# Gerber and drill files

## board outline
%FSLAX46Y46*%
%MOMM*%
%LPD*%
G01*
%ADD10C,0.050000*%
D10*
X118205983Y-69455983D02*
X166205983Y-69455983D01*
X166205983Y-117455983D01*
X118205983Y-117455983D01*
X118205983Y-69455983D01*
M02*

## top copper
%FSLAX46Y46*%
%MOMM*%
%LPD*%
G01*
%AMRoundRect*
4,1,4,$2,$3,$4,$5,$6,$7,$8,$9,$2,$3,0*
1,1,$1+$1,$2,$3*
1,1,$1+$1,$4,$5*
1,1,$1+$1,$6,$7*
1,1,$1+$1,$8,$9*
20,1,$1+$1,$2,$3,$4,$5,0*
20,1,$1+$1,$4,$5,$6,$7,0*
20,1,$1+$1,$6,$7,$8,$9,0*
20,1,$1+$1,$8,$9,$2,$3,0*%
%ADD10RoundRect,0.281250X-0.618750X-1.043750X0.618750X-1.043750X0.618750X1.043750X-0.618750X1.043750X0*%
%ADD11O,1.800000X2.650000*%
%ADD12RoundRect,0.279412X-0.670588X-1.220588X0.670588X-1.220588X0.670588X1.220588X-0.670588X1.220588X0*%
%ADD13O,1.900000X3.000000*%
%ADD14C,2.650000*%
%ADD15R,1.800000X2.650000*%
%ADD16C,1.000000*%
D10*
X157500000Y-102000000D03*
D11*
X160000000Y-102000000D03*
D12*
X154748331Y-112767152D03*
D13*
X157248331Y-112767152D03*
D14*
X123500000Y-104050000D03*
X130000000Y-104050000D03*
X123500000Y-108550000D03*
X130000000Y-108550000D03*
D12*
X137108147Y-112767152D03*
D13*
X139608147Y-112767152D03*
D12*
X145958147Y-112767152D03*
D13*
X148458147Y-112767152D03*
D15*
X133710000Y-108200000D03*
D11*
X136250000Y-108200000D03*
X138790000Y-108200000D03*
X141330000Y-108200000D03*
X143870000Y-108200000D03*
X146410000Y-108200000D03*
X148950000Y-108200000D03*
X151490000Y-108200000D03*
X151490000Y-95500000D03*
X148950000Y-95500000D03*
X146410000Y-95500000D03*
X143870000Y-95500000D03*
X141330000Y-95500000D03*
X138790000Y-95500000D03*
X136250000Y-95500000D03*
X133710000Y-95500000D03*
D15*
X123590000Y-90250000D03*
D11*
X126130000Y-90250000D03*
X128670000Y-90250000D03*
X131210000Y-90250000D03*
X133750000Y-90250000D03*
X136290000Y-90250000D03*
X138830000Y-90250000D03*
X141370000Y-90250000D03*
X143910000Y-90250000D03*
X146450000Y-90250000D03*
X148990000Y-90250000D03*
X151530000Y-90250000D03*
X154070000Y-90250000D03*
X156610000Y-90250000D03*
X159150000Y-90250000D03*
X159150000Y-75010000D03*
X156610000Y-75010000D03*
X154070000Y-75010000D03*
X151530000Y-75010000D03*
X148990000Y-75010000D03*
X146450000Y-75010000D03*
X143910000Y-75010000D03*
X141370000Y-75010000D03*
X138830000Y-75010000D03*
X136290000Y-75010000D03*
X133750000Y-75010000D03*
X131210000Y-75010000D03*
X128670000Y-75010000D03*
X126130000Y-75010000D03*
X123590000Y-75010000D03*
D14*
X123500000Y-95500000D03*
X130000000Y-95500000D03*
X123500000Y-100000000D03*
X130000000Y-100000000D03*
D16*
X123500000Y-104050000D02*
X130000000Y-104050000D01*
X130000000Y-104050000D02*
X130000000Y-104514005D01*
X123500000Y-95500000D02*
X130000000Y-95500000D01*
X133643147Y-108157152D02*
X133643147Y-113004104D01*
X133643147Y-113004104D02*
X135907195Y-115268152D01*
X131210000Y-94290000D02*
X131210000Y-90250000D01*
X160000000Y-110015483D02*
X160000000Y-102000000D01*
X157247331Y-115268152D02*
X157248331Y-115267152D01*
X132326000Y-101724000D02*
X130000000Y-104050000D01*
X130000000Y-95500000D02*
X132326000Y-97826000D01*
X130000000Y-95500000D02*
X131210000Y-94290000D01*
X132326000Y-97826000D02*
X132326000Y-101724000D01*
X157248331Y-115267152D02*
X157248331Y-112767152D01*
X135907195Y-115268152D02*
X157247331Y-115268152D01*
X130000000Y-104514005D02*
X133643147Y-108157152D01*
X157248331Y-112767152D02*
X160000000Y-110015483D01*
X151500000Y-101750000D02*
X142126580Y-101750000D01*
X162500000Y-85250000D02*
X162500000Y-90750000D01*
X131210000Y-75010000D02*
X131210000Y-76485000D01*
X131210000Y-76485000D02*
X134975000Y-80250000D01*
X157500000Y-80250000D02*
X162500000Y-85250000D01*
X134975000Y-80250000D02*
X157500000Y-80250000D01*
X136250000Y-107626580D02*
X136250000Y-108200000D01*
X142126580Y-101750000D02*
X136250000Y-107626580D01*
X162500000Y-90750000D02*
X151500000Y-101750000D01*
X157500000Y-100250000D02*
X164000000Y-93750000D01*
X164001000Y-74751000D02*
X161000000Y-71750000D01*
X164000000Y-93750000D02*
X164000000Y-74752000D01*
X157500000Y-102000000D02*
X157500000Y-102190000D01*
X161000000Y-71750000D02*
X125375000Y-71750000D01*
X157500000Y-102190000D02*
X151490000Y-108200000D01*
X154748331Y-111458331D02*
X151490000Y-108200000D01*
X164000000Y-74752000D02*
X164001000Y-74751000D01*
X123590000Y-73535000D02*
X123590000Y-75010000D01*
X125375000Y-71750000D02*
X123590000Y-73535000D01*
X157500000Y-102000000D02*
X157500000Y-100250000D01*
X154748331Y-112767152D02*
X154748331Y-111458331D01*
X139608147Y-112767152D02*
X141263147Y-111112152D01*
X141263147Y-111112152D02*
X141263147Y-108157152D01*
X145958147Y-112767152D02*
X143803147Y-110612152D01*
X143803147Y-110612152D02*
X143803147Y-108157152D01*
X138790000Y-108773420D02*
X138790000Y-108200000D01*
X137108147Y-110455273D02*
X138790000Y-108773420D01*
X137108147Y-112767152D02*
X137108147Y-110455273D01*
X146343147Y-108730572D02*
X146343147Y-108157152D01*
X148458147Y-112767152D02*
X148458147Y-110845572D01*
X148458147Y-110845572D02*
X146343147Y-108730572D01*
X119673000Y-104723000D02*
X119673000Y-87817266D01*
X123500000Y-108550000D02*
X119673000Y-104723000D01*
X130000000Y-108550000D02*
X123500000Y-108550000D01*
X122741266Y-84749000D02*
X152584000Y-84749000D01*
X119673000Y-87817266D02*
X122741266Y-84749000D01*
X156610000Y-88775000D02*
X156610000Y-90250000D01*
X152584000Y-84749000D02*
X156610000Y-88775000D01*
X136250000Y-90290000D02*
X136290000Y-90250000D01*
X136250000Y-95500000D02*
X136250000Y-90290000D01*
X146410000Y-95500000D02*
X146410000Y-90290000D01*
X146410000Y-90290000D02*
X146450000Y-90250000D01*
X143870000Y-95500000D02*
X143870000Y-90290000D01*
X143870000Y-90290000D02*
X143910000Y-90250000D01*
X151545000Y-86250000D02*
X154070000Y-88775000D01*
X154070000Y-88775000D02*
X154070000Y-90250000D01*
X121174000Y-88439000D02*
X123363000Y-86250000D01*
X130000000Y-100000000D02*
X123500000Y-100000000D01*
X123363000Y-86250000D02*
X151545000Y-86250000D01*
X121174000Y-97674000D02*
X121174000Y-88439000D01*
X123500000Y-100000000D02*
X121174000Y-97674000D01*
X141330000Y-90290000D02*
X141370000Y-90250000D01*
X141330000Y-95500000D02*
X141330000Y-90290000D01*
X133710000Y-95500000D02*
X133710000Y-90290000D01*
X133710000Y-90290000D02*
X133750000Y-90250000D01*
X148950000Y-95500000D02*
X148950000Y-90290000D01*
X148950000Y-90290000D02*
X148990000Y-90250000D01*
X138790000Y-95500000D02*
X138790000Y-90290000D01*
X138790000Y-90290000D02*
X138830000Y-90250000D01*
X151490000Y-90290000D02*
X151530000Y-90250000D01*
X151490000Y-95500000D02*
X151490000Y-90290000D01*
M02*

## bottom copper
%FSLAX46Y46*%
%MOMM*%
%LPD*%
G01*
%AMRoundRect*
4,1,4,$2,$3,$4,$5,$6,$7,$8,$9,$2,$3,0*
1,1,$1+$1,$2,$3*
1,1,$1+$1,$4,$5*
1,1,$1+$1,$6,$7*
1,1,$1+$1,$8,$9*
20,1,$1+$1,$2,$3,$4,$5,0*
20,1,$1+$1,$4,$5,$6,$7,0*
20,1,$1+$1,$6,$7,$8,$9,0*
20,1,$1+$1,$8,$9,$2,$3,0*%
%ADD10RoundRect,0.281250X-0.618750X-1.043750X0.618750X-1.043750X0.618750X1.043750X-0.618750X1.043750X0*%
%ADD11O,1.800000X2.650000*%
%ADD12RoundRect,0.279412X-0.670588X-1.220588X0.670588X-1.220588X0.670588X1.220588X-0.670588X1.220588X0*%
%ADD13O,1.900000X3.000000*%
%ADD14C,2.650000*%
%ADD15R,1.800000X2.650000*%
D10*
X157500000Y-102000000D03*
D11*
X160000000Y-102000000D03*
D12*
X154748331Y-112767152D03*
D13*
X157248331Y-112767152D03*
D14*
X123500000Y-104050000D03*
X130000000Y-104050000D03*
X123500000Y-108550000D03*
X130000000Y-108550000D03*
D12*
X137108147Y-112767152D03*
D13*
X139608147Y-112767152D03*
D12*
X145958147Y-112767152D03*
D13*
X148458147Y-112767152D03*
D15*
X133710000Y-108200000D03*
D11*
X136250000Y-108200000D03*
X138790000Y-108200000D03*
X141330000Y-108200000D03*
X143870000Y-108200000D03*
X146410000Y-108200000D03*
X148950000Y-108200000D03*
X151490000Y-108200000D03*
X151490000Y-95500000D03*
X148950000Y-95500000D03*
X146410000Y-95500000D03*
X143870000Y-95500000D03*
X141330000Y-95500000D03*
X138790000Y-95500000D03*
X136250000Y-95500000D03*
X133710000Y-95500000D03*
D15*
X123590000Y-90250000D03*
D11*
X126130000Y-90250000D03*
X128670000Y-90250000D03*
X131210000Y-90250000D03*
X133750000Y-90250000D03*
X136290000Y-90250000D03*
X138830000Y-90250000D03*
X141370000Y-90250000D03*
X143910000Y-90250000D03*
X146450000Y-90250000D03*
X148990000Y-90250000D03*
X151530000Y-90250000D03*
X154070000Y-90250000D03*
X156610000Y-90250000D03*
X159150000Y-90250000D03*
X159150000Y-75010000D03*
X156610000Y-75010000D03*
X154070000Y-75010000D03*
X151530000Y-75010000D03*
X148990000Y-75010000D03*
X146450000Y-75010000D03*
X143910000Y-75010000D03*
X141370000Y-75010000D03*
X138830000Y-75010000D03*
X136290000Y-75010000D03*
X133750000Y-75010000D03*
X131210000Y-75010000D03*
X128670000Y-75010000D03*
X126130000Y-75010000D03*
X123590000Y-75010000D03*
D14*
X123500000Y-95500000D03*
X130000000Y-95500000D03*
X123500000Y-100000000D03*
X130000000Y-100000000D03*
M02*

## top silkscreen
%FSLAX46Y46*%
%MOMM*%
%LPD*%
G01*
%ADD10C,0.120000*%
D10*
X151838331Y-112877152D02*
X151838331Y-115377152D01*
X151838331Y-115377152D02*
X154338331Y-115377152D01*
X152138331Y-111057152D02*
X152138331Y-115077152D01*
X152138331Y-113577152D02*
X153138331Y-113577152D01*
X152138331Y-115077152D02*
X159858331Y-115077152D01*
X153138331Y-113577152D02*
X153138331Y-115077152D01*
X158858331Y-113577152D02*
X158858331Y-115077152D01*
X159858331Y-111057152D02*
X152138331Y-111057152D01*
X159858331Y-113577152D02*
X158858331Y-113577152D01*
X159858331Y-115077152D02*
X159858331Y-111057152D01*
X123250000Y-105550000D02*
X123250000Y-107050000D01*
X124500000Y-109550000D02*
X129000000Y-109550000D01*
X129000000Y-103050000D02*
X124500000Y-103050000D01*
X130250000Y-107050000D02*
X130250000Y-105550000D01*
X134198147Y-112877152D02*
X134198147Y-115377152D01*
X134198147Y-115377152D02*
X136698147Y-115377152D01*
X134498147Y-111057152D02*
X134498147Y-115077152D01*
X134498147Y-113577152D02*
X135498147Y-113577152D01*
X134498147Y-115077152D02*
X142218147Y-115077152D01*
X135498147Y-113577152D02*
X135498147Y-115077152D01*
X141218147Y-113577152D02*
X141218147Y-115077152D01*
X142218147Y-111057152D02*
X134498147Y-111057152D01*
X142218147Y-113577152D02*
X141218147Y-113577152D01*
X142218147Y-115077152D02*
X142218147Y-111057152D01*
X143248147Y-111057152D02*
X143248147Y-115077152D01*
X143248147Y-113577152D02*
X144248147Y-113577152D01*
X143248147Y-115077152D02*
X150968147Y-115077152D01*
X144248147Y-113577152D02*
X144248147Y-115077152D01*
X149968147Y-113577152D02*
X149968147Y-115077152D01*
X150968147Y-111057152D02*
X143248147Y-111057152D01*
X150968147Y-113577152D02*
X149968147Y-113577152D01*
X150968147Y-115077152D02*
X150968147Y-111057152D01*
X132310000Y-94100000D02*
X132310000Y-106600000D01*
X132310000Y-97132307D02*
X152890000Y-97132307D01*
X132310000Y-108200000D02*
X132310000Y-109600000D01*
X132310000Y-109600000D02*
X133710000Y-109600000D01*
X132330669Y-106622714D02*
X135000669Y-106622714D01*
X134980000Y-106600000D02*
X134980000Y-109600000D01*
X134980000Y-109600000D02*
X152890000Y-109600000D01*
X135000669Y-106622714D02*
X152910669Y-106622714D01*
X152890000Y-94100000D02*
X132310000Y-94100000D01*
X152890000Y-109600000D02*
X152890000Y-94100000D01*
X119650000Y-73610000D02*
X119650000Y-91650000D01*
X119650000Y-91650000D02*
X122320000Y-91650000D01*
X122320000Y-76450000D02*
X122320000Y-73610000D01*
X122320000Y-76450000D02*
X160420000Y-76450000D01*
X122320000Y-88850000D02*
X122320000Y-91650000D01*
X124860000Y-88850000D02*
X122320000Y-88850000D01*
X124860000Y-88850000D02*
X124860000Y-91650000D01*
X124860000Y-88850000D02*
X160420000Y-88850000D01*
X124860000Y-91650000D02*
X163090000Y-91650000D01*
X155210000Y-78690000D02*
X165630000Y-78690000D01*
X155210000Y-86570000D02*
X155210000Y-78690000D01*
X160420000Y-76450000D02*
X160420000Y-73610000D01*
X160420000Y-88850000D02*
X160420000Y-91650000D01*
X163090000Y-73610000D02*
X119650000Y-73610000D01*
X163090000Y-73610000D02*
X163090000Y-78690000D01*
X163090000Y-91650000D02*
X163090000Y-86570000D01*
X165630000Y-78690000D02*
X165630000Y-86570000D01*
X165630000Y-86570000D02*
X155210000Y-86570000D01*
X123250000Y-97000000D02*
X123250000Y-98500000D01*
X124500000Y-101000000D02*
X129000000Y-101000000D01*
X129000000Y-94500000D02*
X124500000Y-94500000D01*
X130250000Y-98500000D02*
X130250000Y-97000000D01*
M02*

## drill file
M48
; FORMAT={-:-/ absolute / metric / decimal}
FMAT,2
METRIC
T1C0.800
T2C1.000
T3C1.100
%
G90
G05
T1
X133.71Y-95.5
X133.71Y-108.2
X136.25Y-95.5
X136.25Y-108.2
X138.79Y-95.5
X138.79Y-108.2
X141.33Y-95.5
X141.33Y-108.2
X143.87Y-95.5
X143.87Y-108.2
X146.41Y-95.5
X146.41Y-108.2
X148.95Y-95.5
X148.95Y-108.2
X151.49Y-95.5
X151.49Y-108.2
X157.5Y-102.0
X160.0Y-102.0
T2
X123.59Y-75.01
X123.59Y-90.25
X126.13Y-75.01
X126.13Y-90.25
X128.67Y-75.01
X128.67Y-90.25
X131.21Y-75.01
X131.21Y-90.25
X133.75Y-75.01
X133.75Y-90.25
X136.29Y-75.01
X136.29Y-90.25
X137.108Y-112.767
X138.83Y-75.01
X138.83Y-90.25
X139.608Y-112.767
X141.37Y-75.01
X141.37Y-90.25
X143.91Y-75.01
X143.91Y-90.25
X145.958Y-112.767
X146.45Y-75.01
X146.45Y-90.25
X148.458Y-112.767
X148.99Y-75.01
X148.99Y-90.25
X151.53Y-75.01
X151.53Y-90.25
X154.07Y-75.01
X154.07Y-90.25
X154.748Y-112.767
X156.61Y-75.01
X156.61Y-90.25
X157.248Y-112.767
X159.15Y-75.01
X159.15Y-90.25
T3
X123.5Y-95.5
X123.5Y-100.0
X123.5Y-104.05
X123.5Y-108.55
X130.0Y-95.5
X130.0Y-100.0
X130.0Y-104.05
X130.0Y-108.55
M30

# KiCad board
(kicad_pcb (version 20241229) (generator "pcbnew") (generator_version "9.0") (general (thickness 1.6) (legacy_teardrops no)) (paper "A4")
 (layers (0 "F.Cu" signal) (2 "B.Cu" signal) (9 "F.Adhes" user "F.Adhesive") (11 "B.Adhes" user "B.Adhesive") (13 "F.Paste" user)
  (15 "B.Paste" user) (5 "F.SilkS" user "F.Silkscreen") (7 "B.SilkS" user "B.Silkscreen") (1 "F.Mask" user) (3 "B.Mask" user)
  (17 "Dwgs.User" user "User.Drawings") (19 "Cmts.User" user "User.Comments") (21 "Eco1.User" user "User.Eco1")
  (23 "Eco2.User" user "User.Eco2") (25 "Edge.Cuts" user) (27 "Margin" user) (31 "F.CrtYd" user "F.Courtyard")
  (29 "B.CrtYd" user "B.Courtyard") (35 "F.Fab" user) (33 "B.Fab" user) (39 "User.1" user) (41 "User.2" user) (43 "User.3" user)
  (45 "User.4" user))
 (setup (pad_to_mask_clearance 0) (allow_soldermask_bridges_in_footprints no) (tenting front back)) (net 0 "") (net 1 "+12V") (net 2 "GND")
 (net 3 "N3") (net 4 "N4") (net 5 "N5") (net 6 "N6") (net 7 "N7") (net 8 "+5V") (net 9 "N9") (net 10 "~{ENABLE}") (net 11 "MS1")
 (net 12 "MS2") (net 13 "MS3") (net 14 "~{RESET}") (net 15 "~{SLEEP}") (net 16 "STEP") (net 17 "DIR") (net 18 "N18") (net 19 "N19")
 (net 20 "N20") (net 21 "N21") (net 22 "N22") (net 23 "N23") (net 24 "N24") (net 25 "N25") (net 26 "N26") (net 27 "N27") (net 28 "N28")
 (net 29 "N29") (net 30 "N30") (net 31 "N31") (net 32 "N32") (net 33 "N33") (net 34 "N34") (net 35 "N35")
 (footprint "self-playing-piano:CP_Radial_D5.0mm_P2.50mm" (layer "F.Cu") (at 157.5 102)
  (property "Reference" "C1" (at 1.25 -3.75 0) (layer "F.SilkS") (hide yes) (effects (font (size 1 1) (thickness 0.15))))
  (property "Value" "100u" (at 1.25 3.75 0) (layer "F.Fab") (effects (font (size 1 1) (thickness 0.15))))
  (pad "1" thru_hole roundrect (at 0 0) (size 1.8 2.65) (drill 0.8) (layers "*.Cu" "*.Mask") (remove_unused_layers no)
   (roundrect_rratio 0.15625) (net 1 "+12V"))
  (pad "2" thru_hole oval (at 2.5 0) (size 1.8 2.65) (drill 0.8) (layers "*.Cu" "*.Mask") (remove_unused_layers no) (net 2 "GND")))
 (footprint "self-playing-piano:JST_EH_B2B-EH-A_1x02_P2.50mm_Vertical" (layer "F.Cu") (at 154.748331 112.767152)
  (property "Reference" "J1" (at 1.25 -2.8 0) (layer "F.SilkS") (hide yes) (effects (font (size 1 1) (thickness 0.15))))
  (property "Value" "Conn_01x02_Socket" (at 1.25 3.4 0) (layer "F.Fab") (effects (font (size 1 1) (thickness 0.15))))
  (fp_line (start -2.91 0.11) (end -2.91 2.61) (stroke (width 0.12) (type solid)) (layer "F.SilkS"))
  (fp_line (start -2.91 2.61) (end -0.41 2.61) (stroke (width 0.12) (type solid)) (layer "F.SilkS"))
  (fp_line (start -2.61 -1.71) (end -2.61 2.31) (stroke (width 0.12) (type solid)) (layer "F.SilkS"))
  (fp_line (start -2.61 0.81) (end -1.61 0.81) (stroke (width 0.12) (type solid)) (layer "F.SilkS"))
  (fp_line (start -2.61 2.31) (end 5.11 2.31) (stroke (width 0.12) (type solid)) (layer "F.SilkS"))
  (fp_line (start -1.61 0.81) (end -1.61 2.31) (stroke (width 0.12) (type solid)) (layer "F.SilkS"))
  (fp_line (start 4.11 0.81) (end 4.11 2.31) (stroke (width 0.12) (type solid)) (layer "F.SilkS"))
  (fp_line (start 5.11 -1.71) (end -2.61 -1.71) (stroke (width 0.12) (type solid)) (layer "F.SilkS"))
  (fp_line (start 5.11 0.81) (end 4.11 0.81) (stroke (width 0.12) (type solid)) (layer "F.SilkS"))
  (fp_line (start 5.11 2.31) (end 5.11 -1.71) (stroke (width 0.12) (type solid)) (layer "F.SilkS"))
  (pad "1" thru_hole roundrect (at 0 0) (size 1.9 3) (drill 1) (layers "*.Cu" "*.Mask") (remove_unused_layers no)
   (roundrect_rratio 0.147059) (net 1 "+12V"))
  (pad "2" thru_hole oval (at 2.5 0) (size 1.9 3) (drill 1) (layers "*.Cu" "*.Mask") (remove_unused_layers no) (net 2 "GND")))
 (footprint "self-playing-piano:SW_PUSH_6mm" (layer "F.Cu") (at 123.5 104.05)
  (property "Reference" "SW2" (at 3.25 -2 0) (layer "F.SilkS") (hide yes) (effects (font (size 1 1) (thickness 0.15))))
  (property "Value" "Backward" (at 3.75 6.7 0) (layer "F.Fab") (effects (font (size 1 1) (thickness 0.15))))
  (fp_line (start -0.25 1.5) (end -0.25 3) (stroke (width 0.12) (type solid)) (layer "F.SilkS"))
  (fp_line (start 1 5.5) (end 5.5 5.5) (stroke (width 0.12) (type solid)) (layer "F.SilkS"))
  (fp_line (start 5.5 -1) (end 1 -1) (stroke (width 0.12) (type solid)) (layer "F.SilkS"))
  (fp_line (start 6.75 3) (end 6.75 1.5) (stroke (width 0.12) (type solid)) (layer "F.SilkS"))
  (pad "1" thru_hole circle (at 0 0 90) (size 2.65 2.65) (drill 1.1) (layers "*.Cu" "*.Mask") (remove_unused_layers no) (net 2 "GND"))
  (pad "1" thru_hole circle (at 6.5 0 90) (size 2.65 2.65) (drill 1.1) (layers "*.Cu" "*.Mask") (remove_unused_layers no) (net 2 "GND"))
  (pad "2" thru_hole circle (at 0 4.5 90) (size 2.65 2.65) (drill 1.1) (layers "*.Cu" "*.Mask") (remove_unused_layers no) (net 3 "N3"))
  (pad "2" thru_hole circle (at 6.5 4.5 90) (size 2.65 2.65) (drill 1.1) (layers "*.Cu" "*.Mask") (remove_unused_layers no) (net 3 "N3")))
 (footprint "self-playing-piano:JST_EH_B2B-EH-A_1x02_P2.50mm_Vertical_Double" (layer "F.Cu") (at 137.108147 112.767152)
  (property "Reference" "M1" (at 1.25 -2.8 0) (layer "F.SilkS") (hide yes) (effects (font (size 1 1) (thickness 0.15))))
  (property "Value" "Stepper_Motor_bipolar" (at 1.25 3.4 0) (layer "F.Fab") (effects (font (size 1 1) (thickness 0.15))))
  (fp_line (start -2.91 0.11) (end -2.91 2.61) (stroke (width 0.12) (type solid)) (layer "F.SilkS"))
  (fp_line (start -2.91 2.61) (end -0.41 2.61) (stroke (width 0.12) (type solid)) (layer "F.SilkS"))
  (fp_line (start -2.61 -1.71) (end -2.61 2.31) (stroke (width 0.12) (type solid)) (layer "F.SilkS"))
  (fp_line (start -2.61 0.81) (end -1.61 0.81) (stroke (width 0.12) (type solid)) (layer "F.SilkS"))
  (fp_line (start -2.61 2.31) (end 5.11 2.31) (stroke (width 0.12) (type solid)) (layer "F.SilkS"))
  (fp_line (start -1.61 0.81) (end -1.61 2.31) (stroke (width 0.12) (type solid)) (layer "F.SilkS"))
  (fp_line (start 4.11 0.81) (end 4.11 2.31) (stroke (width 0.12) (type solid)) (layer "F.SilkS"))
  (fp_line (start 5.11 -1.71) (end -2.61 -1.71) (stroke (width 0.12) (type solid)) (layer "F.SilkS"))
  (fp_line (start 5.11 0.81) (end 4.11 0.81) (stroke (width 0.12) (type solid)) (layer "F.SilkS"))
  (fp_line (start 5.11 2.31) (end 5.11 -1.71) (stroke (width 0.12) (type solid)) (layer "F.SilkS"))
  (fp_line (start 6.14 -1.71) (end 6.14 2.31) (stroke (width 0.12) (type solid)) (layer "F.SilkS"))
  (fp_line (start 6.14 0.81) (end 7.14 0.81) (stroke (width 0.12) (type solid)) (layer "F.SilkS"))
  (fp_line (start 6.14 2.31) (end 13.86 2.31) (stroke (width 0.12) (type solid)) (layer "F.SilkS"))
  (fp_line (start 7.14 0.81) (end 7.14 2.31) (stroke (width 0.12) (type solid)) (layer "F.SilkS"))
  (fp_line (start 12.86 0.81) (end 12.86 2.31) (stroke (width 0.12) (type solid)) (layer "F.SilkS"))
  (fp_line (start 13.86 -1.71) (end 6.14 -1.71) (stroke (width 0.12) (type solid)) (layer "F.SilkS"))
  (fp_line (start 13.86 0.81) (end 12.86 0.81) (stroke (width 0.12) (type solid)) (layer "F.SilkS"))
  (fp_line (start 13.86 2.31) (end 13.86 -1.71) (stroke (width 0.12) (type solid)) (layer "F.SilkS"))
  (pad "1" thru_hole roundrect (at 0 0) (size 1.9 3) (drill 1) (layers "*.Cu" "*.Mask") (remove_unused_layers no)
   (roundrect_rratio 0.147059) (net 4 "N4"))
  (pad "2" thru_hole oval (at 2.5 0) (size 1.9 3) (drill 1) (layers "*.Cu" "*.Mask") (remove_unused_layers no) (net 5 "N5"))
  (pad "3" thru_hole roundrect (at 8.85 0) (size 1.9 3) (drill 1) (layers "*.Cu" "*.Mask") (remove_unused_layers no)
   (roundrect_rratio 0.147059) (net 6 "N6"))
  (pad "4" thru_hole oval (at 11.35 0) (size 1.9 3) (drill 1) (layers "*.Cu" "*.Mask") (remove_unused_layers no) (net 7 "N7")))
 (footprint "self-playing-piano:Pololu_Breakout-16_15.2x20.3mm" (layer "F.Cu") (at 133.71 108.2 90)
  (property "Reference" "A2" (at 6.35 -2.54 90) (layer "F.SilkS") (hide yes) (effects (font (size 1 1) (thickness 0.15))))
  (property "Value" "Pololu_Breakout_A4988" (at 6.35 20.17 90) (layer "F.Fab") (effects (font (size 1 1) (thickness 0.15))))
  (fp_line (start 14.1 -1.4) (end 1.6 -1.4) (stroke (width 0.12) (type solid)) (layer "F.SilkS"))
  (fp_line (start 11.067693 -1.4) (end 11.067693 19.18) (stroke (width 0.12) (type solid)) (layer "F.SilkS"))
  (fp_line (start 0 -1.4) (end -1.4 -1.4) (stroke (width 0.12) (type solid)) (layer "F.SilkS"))
  (fp_line (start -1.4 -1.4) (end -1.4 0) (stroke (width 0.12) (type solid)) (layer "F.SilkS"))
  (fp_line (start 1.577286 -1.379331) (end 1.577286 1.290669) (stroke (width 0.12) (type solid)) (layer "F.SilkS"))
  (fp_line (start 1.6 1.27) (end -1.4 1.27) (stroke (width 0.12) (type solid)) (layer "F.SilkS"))
  (fp_line (start -1.4 1.27) (end -1.4 19.18) (stroke (width 0.12) (type solid)) (layer "F.SilkS"))
  (fp_line (start 1.577286 1.290669) (end 1.577286 19.200669) (stroke (width 0.12) (type solid)) (layer "F.SilkS"))
  (fp_line (start 14.1 19.18) (end 14.1 -1.4) (stroke (width 0.12) (type solid)) (layer "F.SilkS"))
  (fp_line (start -1.4 19.18) (end 14.1 19.18) (stroke (width 0.12) (type solid)) (layer "F.SilkS"))
  (pad "1" thru_hole rect (at 0 0 90) (size 2.65 1.8) (drill 0.8) (layers "*.Cu" "*.Mask") (remove_unused_layers no) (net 2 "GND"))
  (pad "2" thru_hole oval (at 0 2.54 90) (size 2.65 1.8) (drill 0.8) (layers "*.Cu" "*.Mask") (remove_unused_layers no) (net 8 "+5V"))
  (pad "3" thru_hole oval (at 0 5.08 90) (size 2.65 1.8) (drill 0.8) (layers "*.Cu" "*.Mask") (remove_unused_layers no) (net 4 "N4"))
  (pad "4" thru_hole oval (at 0 7.62 90) (size 2.65 1.8) (drill 0.8) (layers "*.Cu" "*.Mask") (remove_unused_layers no) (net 5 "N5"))
  (pad "5" thru_hole oval (at 0 10.16 90) (size 2.65 1.8) (drill 0.8) (layers "*.Cu" "*.Mask") (remove_unused_layers no) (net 6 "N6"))
  (pad "6" thru_hole oval (at 0 12.7 90) (size 2.65 1.8) (drill 0.8) (layers "*.Cu" "*.Mask") (remove_unused_layers no) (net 7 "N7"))
  (pad "7" thru_hole oval (at 0 15.24 90) (size 2.65 1.8) (drill 0.8) (layers "*.Cu" "*.Mask") (remove_unused_layers no) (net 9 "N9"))
  (pad "8" thru_hole oval (at 0 17.78 90) (size 2.65 1.8) (drill 0.8) (layers "*.Cu" "*.Mask") (remove_unused_layers no) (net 1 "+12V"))
  (pad "9" thru_hole oval (at 12.7 17.78 90) (size 2.65 1.8) (drill 0.8) (layers "*.Cu" "*.Mask") (remove_unused_layers no)
   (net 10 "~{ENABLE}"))
  (pad "10" thru_hole oval (at 12.7 15.24 90) (size 2.65 1.8) (drill 0.8) (layers "*.Cu" "*.Mask") (remove_unused_layers no) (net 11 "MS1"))
  (pad "11" thru_hole oval (at 12.7 12.7 90) (size 2.65 1.8) (drill 0.8) (layers "*.Cu" "*.Mask") (remove_unused_layers no) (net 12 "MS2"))
  (pad "12" thru_hole oval (at 12.7 10.16 90) (size 2.65 1.8) (drill 0.8) (layers "*.Cu" "*.Mask") (remove_unused_layers no) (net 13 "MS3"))
  (pad "13" thru_hole oval (at 12.7 7.62 90) (size 2.65 1.8) (drill 0.8) (layers "*.Cu" "*.Mask") (remove_unused_layers no)
   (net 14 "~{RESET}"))
  (pad "14" thru_hole oval (at 12.7 5.08 90) (size 2.65 1.8) (drill 0.8) (layers "*.Cu" "*.Mask") (remove_unused_layers no)
   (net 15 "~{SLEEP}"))
  (pad "15" thru_hole oval (at 12.7 2.54 90) (size 2.65 1.8) (drill 0.8) (layers "*.Cu" "*.Mask") (remove_unused_layers no) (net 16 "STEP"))
  (pad "16" thru_hole oval (at 12.7 0 90) (size 2.65 1.8) (drill 0.8) (layers "*.Cu" "*.Mask") (remove_unused_layers no) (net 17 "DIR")))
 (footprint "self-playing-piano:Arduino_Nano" (layer "F.Cu") (at 123.59 90.25 90)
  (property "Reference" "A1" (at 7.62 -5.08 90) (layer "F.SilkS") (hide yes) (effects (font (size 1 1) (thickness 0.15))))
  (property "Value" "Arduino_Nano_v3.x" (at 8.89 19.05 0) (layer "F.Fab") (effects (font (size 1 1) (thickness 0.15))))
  (fp_line (start 16.64 -3.94) (end -1.4 -3.94) (stroke (width 0.12) (type solid)) (layer "F.SilkS"))
  (fp_line (start -1.4 -3.94) (end -1.4 -1.27) (stroke (width 0.12) (type solid)) (layer "F.SilkS"))
  (fp_line (start 13.8 -1.27) (end 16.64 -1.27) (stroke (width 0.12) (type solid)) (layer "F.SilkS"))
  (fp_line (start 13.8 -1.27) (end 13.8 36.83) (stroke (width 0.12) (type solid)) (layer "F.SilkS"))
  (fp_line (start 1.4 -1.27) (end -1.4 -1.27) (stroke (width 0.12) (type solid)) (layer "F.SilkS"))
  (fp_line (start 1.4 1.27) (end 1.4 -1.27) (stroke (width 0.12) (type solid)) (layer "F.SilkS"))
  (fp_line (start 1.4 1.27) (end -1.4 1.27) (stroke (width 0.12) (type solid)) (layer "F.SilkS"))
  (fp_line (start 1.4 1.27) (end 1.4 36.83) (stroke (width 0.12) (type solid)) (layer "F.SilkS"))
  (fp_line (start -1.4 1.27) (end -1.4 39.5) (stroke (width 0.12) (type solid)) (layer "F.SilkS"))
  (fp_line (start 11.56 31.62) (end 11.56 42.04) (stroke (width 0.12) (type solid)) (layer "F.SilkS"))
  (fp_line (start 3.68 31.62) (end 11.56 31.62) (stroke (width 0.12) (type solid)) (layer "F.SilkS"))
  (fp_line (start 13.8 36.83) (end 16.64 36.83) (stroke (width 0.12) (type solid)) (layer "F.SilkS"))
  (fp_line (start 1.4 36.83) (end -1.4 36.83) (stroke (width 0.12) (type solid)) (layer "F.SilkS"))
  (fp_line (start 16.64 39.5) (end 16.64 -3.94) (stroke (width 0.12) (type solid)) (layer "F.SilkS"))
  (fp_line (start 16.64 39.5) (end 11.56 39.5) (stroke (width 0.12) (type solid)) (layer "F.SilkS"))
  (fp_line (start -1.4 39.5) (end 3.68 39.5) (stroke (width 0.12) (type solid)) (layer "F.SilkS"))
  (fp_line (start 11.56 42.04) (end 3.68 42.04) (stroke (width 0.12) (type solid)) (layer "F.SilkS"))
  (fp_line (start 3.68 42.04) (end 3.68 31.62) (stroke (width 0.12) (type solid)) (layer "F.SilkS"))
  (pad "1" thru_hole rect (at 0 0 90) (size 2.65 1.8) (drill 1) (layers "*.Cu" "*.Mask") (remove_unused_layers no) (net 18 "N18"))
  (pad "2" thru_hole oval (at 0 2.54 90) (size 2.65 1.8) (drill 1) (layers "*.Cu" "*.Mask") (remove_unused_layers no) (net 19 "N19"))
  (pad "3" thru_hole oval (at 0 5.08 90) (size 2.65 1.8) (drill 1) (layers "*.Cu" "*.Mask") (remove_unused_layers no) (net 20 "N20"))
  (pad "4" thru_hole oval (at 0 7.62 90) (size 2.65 1.8) (drill 1) (layers "*.Cu" "*.Mask") (remove_unused_layers no) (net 2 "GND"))
  (pad "5" thru_hole oval (at 0 10.16 90) (size 2.65 1.8) (drill 1) (layers "*.Cu" "*.Mask") (remove_unused_layers no) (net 17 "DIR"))
  (pad "6" thru_hole oval (at 0 12.7 90) (size 2.65 1.8) (drill 1) (layers "*.Cu" "*.Mask") (remove_unused_layers no) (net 16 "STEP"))
  (pad "7" thru_hole oval (at 0 15.24 90) (size 2.65 1.8) (drill 1) (layers "*.Cu" "*.Mask") (remove_unused_layers no) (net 15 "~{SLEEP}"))
  (pad "8" thru_hole oval (at 0 17.78 90) (size 2.65 1.8) (drill 1) (layers "*.Cu" "*.Mask") (remove_unused_layers no) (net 14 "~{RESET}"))
  (pad "9" thru_hole oval (at 0 20.32 90) (size 2.65 1.8) (drill 1) (layers "*.Cu" "*.Mask") (remove_unused_layers no) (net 13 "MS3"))
  (pad "10" thru_hole oval (at 0 22.86 90) (size 2.65 1.8) (drill 1) (layers "*.Cu" "*.Mask") (remove_unused_layers no) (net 12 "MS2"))
  (pad "11" thru_hole oval (at 0 25.4 90) (size 2.65 1.8) (drill 1) (layers "*.Cu" "*.Mask") (remove_unused_layers no) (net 11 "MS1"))
  (pad "12" thru_hole oval (at 0 27.94 90) (size 2.65 1.8) (drill 1) (layers "*.Cu" "*.Mask") (remove_unused_layers no) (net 10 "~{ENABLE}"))
  (pad "13" thru_hole oval (at 0 30.48 90) (size 2.65 1.8) (drill 1) (layers "*.Cu" "*.Mask") (remove_unused_layers no) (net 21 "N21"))
  (pad "14" thru_hole oval (at 0 33.02 90) (size 2.65 1.8) (drill 1) (layers "*.Cu" "*.Mask") (remove_unused_layers no) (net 3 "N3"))
  (pad "15" thru_hole oval (at 0 35.56 90) (size 2.65 1.8) (drill 1) (layers "*.Cu" "*.Mask") (remove_unused_layers no) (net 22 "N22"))
  (pad "16" thru_hole oval (at 15.24 35.56 90) (size 2.65 1.8) (drill 1) (layers "*.Cu" "*.Mask") (remove_unused_layers no) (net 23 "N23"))
  (pad "17" thru_hole oval (at 15.24 33.02 90) (size 2.65 1.8) (drill 1) (layers "*.Cu" "*.Mask") (remove_unused_layers no) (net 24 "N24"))
  (pad "18" thru_hole oval (at 15.24 30.48 90) (size 2.65 1.8) (drill 1) (layers "*.Cu" "*.Mask") (remove_unused_layers no) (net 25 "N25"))
  (pad "19" thru_hole oval (at 15.24 27.94 90) (size 2.65 1.8) (drill 1) (layers "*.Cu" "*.Mask") (remove_unused_layers no) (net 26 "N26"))
  (pad "20" thru_hole oval (at 15.24 25.4 90) (size 2.65 1.8) (drill 1) (layers "*.Cu" "*.Mask") (remove_unused_layers no) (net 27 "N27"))
  (pad "21" thru_hole oval (at 15.24 22.86 90) (size 2.65 1.8) (drill 1) (layers "*.Cu" "*.Mask") (remove_unused_layers no) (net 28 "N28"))
  (pad "22" thru_hole oval (at 15.24 20.32 90) (size 2.65 1.8) (drill 1) (layers "*.Cu" "*.Mask") (remove_unused_layers no) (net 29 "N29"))
  (pad "23" thru_hole oval (at 15.24 17.78 90) (size 2.65 1.8) (drill 1) (layers "*.Cu" "*.Mask") (remove_unused_layers no) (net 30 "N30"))
  (pad "24" thru_hole oval (at 15.24 15.24 90) (size 2.65 1.8) (drill 1) (layers "*.Cu" "*.Mask") (remove_unused_layers no) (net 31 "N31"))
  (pad "25" thru_hole oval (at 15.24 12.7 90) (size 2.65 1.8) (drill 1) (layers "*.Cu" "*.Mask") (remove_unused_layers no) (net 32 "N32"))
  (pad "26" thru_hole oval (at 15.24 10.16 90) (size 2.65 1.8) (drill 1) (layers "*.Cu" "*.Mask") (remove_unused_layers no) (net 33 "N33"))
  (pad "27" thru_hole oval (at 15.24 7.62 90) (size 2.65 1.8) (drill 1) (layers "*.Cu" "*.Mask") (remove_unused_layers no) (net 8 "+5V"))
  (pad "28" thru_hole oval (at 15.24 5.08 90) (size 2.65 1.8) (drill 1) (layers "*.Cu" "*.Mask") (remove_unused_layers no) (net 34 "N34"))
  (pad "29" thru_hole oval (at 15.24 2.54 90) (size 2.65 1.8) (drill 1) (layers "*.Cu" "*.Mask") (remove_unused_layers no) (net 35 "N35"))
  (pad "30" thru_hole oval (at 15.24 0 90) (size 2.65 1.8) (drill 1) (layers "*.Cu" "*.Mask") (remove_unused_layers no) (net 1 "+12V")))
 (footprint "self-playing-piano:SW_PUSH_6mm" (layer "F.Cu") (at 123.5 95.5)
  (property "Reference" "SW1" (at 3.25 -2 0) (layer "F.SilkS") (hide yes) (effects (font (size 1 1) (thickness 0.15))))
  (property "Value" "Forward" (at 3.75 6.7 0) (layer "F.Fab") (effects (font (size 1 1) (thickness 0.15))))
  (fp_line (start -0.25 1.5) (end -0.25 3) (stroke (width 0.12) (type solid)) (layer "F.SilkS"))
  (fp_line (start 1 5.5) (end 5.5 5.5) (stroke (width 0.12) (type solid)) (layer "F.SilkS"))
  (fp_line (start 5.5 -1) (end 1 -1) (stroke (width 0.12) (type solid)) (layer "F.SilkS"))
  (fp_line (start 6.75 3) (end 6.75 1.5) (stroke (width 0.12) (type solid)) (layer "F.SilkS"))
  (pad "1" thru_hole circle (at 0 0 90) (size 2.65 2.65) (drill 1.1) (layers "*.Cu" "*.Mask") (remove_unused_layers no) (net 2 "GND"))
  (pad "1" thru_hole circle (at 6.5 0 90) (size 2.65 2.65) (drill 1.1) (layers "*.Cu" "*.Mask") (remove_unused_layers no) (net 2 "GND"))
  (pad "2" thru_hole circle (at 0 4.5 90) (size 2.65 2.65) (drill 1.1) (layers "*.Cu" "*.Mask") (remove_unused_layers no) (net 21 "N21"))
  (pad "2" thru_hole circle (at 6.5 4.5 90) (size 2.65 2.65) (drill 1.1) (layers "*.Cu" "*.Mask") (remove_unused_layers no) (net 21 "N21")))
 (gr_rect (start 118.205983 69.455983) (end 166.205983 117.455983) (stroke (width 0.05) (type default)) (fill no) (layer "Edge.Cuts"))
 (segment (start 123.5 104.05) (end 130 104.05) (width 1) (layer "F.Cu") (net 2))
 (segment (start 130 104.05) (end 130 104.514005) (width 1) (layer "F.Cu") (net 2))
 (segment (start 123.5 95.5) (end 130 95.5) (width 1) (layer "F.Cu") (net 2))
 (segment (start 133.643147 108.157152) (end 133.643147 113.004104) (width 1) (layer "F.Cu") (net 2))
 (segment (start 133.643147 113.004104) (end 135.907195 115.268152) (width 1) (layer "F.Cu") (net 2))
 (segment (start 131.21 94.29) (end 131.21 90.25) (width 1) (layer "F.Cu") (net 2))
 (segment (start 160 110.015483) (end 160 102) (width 1) (layer "F.Cu") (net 2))
 (segment (start 157.247331 115.268152) (end 157.248331 115.267152) (width 1) (layer "F.Cu") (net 2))
 (segment (start 132.326 101.724) (end 130 104.05) (width 1) (layer "F.Cu") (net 2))
 (segment (start 130 95.5) (end 132.326 97.826) (width 1) (layer "F.Cu") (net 2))
 (segment (start 130 95.5) (end 131.21 94.29) (width 1) (layer "F.Cu") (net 2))
 (segment (start 132.326 97.826) (end 132.326 101.724) (width 1) (layer "F.Cu") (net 2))
 (segment (start 157.248331 115.267152) (end 157.248331 112.767152) (width 1) (layer "F.Cu") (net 2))
 (segment (start 135.907195 115.268152) (end 157.247331 115.268152) (width 1) (layer "F.Cu") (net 2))
 (segment (start 130 104.514005) (end 133.643147 108.157152) (width 1) (layer "F.Cu") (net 2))
 (segment (start 157.248331 112.767152) (end 160 110.015483) (width 1) (layer "F.Cu") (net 2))
 (segment (start 151.5 101.75) (end 142.12658 101.75) (width 1) (layer "F.Cu") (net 8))
 (segment (start 162.5 85.25) (end 162.5 90.75) (width 1) (layer "F.Cu") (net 8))
 (segment (start 131.21 75.01) (end 131.21 76.485) (width 1) (layer "F.Cu") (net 8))
 (segment (start 131.21 76.485) (end 134.975 80.25) (width 1) (layer "F.Cu") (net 8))
 (segment (start 157.5 80.25) (end 162.5 85.25) (width 1) (layer "F.Cu") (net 8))
 (segment (start 134.975 80.25) (end 157.5 80.25) (width 1) (layer "F.Cu") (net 8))
 (segment (start 136.25 107.62658) (end 136.25 108.2) (width 1) (layer "F.Cu") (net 8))
 (segment (start 142.12658 101.75) (end 136.25 107.62658) (width 1) (layer "F.Cu") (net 8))
 (segment (start 162.5 90.75) (end 151.5 101.75) (width 1) (layer "F.Cu") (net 8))
 (segment (start 157.5 100.25) (end 164 93.75) (width 1) (layer "F.Cu") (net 1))
 (segment (start 164.001 74.751) (end 161 71.75) (width 1) (layer "F.Cu") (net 1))
 (segment (start 164 93.75) (end 164 74.752) (width 1) (layer "F.Cu") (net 1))
 (segment (start 157.5 102) (end 157.5 102.19) (width 1) (layer "F.Cu") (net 1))
 (segment (start 161 71.75) (end 125.375 71.75) (width 1) (layer "F.Cu") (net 1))
 (segment (start 157.5 102.19) (end 151.49 108.2) (width 1) (layer "F.Cu") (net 1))
 (segment (start 154.748331 111.458331) (end 151.49 108.2) (width 1) (layer "F.Cu") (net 1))
 (segment (start 164 74.752) (end 164.001 74.751) (width 1) (layer "F.Cu") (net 1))
 (segment (start 123.59 73.535) (end 123.59 75.01) (width 1) (layer "F.Cu") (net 1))
 (segment (start 125.375 71.75) (end 123.59 73.535) (width 1) (layer "F.Cu") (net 1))
 (segment (start 157.5 102) (end 157.5 100.25) (width 1) (layer "F.Cu") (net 1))
 (segment (start 154.748331 112.767152) (end 154.748331 111.458331) (width 1) (layer "F.Cu") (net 1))
 (segment (start 139.608147 112.767152) (end 141.263147 111.112152) (width 1) (layer "F.Cu") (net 5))
 (segment (start 141.263147 111.112152) (end 141.263147 108.157152) (width 1) (layer "F.Cu") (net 5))
 (segment (start 145.958147 112.767152) (end 143.803147 110.612152) (width 1) (layer "F.Cu") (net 6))
 (segment (start 143.803147 110.612152) (end 143.803147 108.157152) (width 1) (layer "F.Cu") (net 6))
 (segment (start 138.79 108.77342) (end 138.79 108.2) (width 1) (layer "F.Cu") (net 4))
 (segment (start 137.108147 110.455273) (end 138.79 108.77342) (width 1) (layer "F.Cu") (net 4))
 (segment (start 137.108147 112.767152) (end 137.108147 110.455273) (width 1) (layer "F.Cu") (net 4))
 (segment (start 146.343147 108.730572) (end 146.343147 108.157152) (width 1) (layer "F.Cu") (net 7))
 (segment (start 148.458147 112.767152) (end 148.458147 110.845572) (width 1) (layer "F.Cu") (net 7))
 (segment (start 148.458147 110.845572) (end 146.343147 108.730572) (width 1) (layer "F.Cu") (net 7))
 (segment (start 119.673 104.723) (end 119.673 87.817266) (width 1) (layer "F.Cu") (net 3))
 (segment (start 123.5 108.55) (end 119.673 104.723) (width 1) (layer "F.Cu") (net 3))
 (segment (start 130 108.55) (end 123.5 108.55) (width 1) (layer "F.Cu") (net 3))
 (segment (start 122.741266 84.749) (end 152.584 84.749) (width 1) (layer "F.Cu") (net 3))
 (segment (start 119.673 87.817266) (end 122.741266 84.749) (width 1) (layer "F.Cu") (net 3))
 (segment (start 156.61 88.775) (end 156.61 90.25) (width 1) (layer "F.Cu") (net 3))
 (segment (start 152.584 84.749) (end 156.61 88.775) (width 1) (layer "F.Cu") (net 3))
 (segment (start 136.25 90.29) (end 136.29 90.25) (width 1) (layer "F.Cu") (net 16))
 (segment (start 136.25 95.5) (end 136.25 90.29) (width 1) (layer "F.Cu") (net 16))
 (segment (start 146.41 95.5) (end 146.41 90.29) (width 1) (layer "F.Cu") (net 12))
 (segment (start 146.41 90.29) (end 146.45 90.25) (width 1) (layer "F.Cu") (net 12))
 (segment (start 143.87 95.5) (end 143.87 90.29) (width 1) (layer "F.Cu") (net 13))
 (segment (start 143.87 90.29) (end 143.91 90.25) (width 1) (layer "F.Cu") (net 13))
 (segment (start 151.545 86.25) (end 154.07 88.775) (width 1) (layer "F.Cu") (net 21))
 (segment (start 154.07 88.775) (end 154.07 90.25) (width 1) (layer "F.Cu") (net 21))
 (segment (start 121.174 88.439) (end 123.363 86.25) (width 1) (layer "F.Cu") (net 21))
 (segment (start 130 100) (end 123.5 100) (width 1) (layer "F.Cu") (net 21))
 (segment (start 123.363 86.25) (end 151.545 86.25) (width 1) (layer "F.Cu") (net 21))
 (segment (start 121.174 97.674) (end 121.174 88.439) (width 1) (layer "F.Cu") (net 21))
 (segment (start 123.5 100) (end 121.174 97.674) (width 1) (layer "F.Cu") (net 21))
 (segment (start 141.33 90.29) (end 141.37 90.25) (width 1) (layer "F.Cu") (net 14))
 (segment (start 141.33 95.5) (end 141.33 90.29) (width 1) (layer "F.Cu") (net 14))
 (segment (start 133.71 95.5) (end 133.71 90.29) (width 1) (layer "F.Cu") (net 17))
 (segment (start 133.71 90.29) (end 133.75 90.25) (width 1) (layer "F.Cu") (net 17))
 (segment (start 148.95 95.5) (end 148.95 90.29) (width 1) (layer "F.Cu") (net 11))
 (segment (start 148.95 90.29) (end 148.99 90.25) (width 1) (layer "F.Cu") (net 11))
 (segment (start 138.79 95.5) (end 138.79 90.29) (width 1) (layer "F.Cu") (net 15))
 (segment (start 138.79 90.29) (end 138.83 90.25) (width 1) (layer "F.Cu") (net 15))
 (segment (start 151.49 90.29) (end 151.53 90.25) (width 1) (layer "F.Cu") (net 10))
 (segment (start 151.49 95.5) (end 151.49 90.29) (width 1) (layer "F.Cu") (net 10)))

